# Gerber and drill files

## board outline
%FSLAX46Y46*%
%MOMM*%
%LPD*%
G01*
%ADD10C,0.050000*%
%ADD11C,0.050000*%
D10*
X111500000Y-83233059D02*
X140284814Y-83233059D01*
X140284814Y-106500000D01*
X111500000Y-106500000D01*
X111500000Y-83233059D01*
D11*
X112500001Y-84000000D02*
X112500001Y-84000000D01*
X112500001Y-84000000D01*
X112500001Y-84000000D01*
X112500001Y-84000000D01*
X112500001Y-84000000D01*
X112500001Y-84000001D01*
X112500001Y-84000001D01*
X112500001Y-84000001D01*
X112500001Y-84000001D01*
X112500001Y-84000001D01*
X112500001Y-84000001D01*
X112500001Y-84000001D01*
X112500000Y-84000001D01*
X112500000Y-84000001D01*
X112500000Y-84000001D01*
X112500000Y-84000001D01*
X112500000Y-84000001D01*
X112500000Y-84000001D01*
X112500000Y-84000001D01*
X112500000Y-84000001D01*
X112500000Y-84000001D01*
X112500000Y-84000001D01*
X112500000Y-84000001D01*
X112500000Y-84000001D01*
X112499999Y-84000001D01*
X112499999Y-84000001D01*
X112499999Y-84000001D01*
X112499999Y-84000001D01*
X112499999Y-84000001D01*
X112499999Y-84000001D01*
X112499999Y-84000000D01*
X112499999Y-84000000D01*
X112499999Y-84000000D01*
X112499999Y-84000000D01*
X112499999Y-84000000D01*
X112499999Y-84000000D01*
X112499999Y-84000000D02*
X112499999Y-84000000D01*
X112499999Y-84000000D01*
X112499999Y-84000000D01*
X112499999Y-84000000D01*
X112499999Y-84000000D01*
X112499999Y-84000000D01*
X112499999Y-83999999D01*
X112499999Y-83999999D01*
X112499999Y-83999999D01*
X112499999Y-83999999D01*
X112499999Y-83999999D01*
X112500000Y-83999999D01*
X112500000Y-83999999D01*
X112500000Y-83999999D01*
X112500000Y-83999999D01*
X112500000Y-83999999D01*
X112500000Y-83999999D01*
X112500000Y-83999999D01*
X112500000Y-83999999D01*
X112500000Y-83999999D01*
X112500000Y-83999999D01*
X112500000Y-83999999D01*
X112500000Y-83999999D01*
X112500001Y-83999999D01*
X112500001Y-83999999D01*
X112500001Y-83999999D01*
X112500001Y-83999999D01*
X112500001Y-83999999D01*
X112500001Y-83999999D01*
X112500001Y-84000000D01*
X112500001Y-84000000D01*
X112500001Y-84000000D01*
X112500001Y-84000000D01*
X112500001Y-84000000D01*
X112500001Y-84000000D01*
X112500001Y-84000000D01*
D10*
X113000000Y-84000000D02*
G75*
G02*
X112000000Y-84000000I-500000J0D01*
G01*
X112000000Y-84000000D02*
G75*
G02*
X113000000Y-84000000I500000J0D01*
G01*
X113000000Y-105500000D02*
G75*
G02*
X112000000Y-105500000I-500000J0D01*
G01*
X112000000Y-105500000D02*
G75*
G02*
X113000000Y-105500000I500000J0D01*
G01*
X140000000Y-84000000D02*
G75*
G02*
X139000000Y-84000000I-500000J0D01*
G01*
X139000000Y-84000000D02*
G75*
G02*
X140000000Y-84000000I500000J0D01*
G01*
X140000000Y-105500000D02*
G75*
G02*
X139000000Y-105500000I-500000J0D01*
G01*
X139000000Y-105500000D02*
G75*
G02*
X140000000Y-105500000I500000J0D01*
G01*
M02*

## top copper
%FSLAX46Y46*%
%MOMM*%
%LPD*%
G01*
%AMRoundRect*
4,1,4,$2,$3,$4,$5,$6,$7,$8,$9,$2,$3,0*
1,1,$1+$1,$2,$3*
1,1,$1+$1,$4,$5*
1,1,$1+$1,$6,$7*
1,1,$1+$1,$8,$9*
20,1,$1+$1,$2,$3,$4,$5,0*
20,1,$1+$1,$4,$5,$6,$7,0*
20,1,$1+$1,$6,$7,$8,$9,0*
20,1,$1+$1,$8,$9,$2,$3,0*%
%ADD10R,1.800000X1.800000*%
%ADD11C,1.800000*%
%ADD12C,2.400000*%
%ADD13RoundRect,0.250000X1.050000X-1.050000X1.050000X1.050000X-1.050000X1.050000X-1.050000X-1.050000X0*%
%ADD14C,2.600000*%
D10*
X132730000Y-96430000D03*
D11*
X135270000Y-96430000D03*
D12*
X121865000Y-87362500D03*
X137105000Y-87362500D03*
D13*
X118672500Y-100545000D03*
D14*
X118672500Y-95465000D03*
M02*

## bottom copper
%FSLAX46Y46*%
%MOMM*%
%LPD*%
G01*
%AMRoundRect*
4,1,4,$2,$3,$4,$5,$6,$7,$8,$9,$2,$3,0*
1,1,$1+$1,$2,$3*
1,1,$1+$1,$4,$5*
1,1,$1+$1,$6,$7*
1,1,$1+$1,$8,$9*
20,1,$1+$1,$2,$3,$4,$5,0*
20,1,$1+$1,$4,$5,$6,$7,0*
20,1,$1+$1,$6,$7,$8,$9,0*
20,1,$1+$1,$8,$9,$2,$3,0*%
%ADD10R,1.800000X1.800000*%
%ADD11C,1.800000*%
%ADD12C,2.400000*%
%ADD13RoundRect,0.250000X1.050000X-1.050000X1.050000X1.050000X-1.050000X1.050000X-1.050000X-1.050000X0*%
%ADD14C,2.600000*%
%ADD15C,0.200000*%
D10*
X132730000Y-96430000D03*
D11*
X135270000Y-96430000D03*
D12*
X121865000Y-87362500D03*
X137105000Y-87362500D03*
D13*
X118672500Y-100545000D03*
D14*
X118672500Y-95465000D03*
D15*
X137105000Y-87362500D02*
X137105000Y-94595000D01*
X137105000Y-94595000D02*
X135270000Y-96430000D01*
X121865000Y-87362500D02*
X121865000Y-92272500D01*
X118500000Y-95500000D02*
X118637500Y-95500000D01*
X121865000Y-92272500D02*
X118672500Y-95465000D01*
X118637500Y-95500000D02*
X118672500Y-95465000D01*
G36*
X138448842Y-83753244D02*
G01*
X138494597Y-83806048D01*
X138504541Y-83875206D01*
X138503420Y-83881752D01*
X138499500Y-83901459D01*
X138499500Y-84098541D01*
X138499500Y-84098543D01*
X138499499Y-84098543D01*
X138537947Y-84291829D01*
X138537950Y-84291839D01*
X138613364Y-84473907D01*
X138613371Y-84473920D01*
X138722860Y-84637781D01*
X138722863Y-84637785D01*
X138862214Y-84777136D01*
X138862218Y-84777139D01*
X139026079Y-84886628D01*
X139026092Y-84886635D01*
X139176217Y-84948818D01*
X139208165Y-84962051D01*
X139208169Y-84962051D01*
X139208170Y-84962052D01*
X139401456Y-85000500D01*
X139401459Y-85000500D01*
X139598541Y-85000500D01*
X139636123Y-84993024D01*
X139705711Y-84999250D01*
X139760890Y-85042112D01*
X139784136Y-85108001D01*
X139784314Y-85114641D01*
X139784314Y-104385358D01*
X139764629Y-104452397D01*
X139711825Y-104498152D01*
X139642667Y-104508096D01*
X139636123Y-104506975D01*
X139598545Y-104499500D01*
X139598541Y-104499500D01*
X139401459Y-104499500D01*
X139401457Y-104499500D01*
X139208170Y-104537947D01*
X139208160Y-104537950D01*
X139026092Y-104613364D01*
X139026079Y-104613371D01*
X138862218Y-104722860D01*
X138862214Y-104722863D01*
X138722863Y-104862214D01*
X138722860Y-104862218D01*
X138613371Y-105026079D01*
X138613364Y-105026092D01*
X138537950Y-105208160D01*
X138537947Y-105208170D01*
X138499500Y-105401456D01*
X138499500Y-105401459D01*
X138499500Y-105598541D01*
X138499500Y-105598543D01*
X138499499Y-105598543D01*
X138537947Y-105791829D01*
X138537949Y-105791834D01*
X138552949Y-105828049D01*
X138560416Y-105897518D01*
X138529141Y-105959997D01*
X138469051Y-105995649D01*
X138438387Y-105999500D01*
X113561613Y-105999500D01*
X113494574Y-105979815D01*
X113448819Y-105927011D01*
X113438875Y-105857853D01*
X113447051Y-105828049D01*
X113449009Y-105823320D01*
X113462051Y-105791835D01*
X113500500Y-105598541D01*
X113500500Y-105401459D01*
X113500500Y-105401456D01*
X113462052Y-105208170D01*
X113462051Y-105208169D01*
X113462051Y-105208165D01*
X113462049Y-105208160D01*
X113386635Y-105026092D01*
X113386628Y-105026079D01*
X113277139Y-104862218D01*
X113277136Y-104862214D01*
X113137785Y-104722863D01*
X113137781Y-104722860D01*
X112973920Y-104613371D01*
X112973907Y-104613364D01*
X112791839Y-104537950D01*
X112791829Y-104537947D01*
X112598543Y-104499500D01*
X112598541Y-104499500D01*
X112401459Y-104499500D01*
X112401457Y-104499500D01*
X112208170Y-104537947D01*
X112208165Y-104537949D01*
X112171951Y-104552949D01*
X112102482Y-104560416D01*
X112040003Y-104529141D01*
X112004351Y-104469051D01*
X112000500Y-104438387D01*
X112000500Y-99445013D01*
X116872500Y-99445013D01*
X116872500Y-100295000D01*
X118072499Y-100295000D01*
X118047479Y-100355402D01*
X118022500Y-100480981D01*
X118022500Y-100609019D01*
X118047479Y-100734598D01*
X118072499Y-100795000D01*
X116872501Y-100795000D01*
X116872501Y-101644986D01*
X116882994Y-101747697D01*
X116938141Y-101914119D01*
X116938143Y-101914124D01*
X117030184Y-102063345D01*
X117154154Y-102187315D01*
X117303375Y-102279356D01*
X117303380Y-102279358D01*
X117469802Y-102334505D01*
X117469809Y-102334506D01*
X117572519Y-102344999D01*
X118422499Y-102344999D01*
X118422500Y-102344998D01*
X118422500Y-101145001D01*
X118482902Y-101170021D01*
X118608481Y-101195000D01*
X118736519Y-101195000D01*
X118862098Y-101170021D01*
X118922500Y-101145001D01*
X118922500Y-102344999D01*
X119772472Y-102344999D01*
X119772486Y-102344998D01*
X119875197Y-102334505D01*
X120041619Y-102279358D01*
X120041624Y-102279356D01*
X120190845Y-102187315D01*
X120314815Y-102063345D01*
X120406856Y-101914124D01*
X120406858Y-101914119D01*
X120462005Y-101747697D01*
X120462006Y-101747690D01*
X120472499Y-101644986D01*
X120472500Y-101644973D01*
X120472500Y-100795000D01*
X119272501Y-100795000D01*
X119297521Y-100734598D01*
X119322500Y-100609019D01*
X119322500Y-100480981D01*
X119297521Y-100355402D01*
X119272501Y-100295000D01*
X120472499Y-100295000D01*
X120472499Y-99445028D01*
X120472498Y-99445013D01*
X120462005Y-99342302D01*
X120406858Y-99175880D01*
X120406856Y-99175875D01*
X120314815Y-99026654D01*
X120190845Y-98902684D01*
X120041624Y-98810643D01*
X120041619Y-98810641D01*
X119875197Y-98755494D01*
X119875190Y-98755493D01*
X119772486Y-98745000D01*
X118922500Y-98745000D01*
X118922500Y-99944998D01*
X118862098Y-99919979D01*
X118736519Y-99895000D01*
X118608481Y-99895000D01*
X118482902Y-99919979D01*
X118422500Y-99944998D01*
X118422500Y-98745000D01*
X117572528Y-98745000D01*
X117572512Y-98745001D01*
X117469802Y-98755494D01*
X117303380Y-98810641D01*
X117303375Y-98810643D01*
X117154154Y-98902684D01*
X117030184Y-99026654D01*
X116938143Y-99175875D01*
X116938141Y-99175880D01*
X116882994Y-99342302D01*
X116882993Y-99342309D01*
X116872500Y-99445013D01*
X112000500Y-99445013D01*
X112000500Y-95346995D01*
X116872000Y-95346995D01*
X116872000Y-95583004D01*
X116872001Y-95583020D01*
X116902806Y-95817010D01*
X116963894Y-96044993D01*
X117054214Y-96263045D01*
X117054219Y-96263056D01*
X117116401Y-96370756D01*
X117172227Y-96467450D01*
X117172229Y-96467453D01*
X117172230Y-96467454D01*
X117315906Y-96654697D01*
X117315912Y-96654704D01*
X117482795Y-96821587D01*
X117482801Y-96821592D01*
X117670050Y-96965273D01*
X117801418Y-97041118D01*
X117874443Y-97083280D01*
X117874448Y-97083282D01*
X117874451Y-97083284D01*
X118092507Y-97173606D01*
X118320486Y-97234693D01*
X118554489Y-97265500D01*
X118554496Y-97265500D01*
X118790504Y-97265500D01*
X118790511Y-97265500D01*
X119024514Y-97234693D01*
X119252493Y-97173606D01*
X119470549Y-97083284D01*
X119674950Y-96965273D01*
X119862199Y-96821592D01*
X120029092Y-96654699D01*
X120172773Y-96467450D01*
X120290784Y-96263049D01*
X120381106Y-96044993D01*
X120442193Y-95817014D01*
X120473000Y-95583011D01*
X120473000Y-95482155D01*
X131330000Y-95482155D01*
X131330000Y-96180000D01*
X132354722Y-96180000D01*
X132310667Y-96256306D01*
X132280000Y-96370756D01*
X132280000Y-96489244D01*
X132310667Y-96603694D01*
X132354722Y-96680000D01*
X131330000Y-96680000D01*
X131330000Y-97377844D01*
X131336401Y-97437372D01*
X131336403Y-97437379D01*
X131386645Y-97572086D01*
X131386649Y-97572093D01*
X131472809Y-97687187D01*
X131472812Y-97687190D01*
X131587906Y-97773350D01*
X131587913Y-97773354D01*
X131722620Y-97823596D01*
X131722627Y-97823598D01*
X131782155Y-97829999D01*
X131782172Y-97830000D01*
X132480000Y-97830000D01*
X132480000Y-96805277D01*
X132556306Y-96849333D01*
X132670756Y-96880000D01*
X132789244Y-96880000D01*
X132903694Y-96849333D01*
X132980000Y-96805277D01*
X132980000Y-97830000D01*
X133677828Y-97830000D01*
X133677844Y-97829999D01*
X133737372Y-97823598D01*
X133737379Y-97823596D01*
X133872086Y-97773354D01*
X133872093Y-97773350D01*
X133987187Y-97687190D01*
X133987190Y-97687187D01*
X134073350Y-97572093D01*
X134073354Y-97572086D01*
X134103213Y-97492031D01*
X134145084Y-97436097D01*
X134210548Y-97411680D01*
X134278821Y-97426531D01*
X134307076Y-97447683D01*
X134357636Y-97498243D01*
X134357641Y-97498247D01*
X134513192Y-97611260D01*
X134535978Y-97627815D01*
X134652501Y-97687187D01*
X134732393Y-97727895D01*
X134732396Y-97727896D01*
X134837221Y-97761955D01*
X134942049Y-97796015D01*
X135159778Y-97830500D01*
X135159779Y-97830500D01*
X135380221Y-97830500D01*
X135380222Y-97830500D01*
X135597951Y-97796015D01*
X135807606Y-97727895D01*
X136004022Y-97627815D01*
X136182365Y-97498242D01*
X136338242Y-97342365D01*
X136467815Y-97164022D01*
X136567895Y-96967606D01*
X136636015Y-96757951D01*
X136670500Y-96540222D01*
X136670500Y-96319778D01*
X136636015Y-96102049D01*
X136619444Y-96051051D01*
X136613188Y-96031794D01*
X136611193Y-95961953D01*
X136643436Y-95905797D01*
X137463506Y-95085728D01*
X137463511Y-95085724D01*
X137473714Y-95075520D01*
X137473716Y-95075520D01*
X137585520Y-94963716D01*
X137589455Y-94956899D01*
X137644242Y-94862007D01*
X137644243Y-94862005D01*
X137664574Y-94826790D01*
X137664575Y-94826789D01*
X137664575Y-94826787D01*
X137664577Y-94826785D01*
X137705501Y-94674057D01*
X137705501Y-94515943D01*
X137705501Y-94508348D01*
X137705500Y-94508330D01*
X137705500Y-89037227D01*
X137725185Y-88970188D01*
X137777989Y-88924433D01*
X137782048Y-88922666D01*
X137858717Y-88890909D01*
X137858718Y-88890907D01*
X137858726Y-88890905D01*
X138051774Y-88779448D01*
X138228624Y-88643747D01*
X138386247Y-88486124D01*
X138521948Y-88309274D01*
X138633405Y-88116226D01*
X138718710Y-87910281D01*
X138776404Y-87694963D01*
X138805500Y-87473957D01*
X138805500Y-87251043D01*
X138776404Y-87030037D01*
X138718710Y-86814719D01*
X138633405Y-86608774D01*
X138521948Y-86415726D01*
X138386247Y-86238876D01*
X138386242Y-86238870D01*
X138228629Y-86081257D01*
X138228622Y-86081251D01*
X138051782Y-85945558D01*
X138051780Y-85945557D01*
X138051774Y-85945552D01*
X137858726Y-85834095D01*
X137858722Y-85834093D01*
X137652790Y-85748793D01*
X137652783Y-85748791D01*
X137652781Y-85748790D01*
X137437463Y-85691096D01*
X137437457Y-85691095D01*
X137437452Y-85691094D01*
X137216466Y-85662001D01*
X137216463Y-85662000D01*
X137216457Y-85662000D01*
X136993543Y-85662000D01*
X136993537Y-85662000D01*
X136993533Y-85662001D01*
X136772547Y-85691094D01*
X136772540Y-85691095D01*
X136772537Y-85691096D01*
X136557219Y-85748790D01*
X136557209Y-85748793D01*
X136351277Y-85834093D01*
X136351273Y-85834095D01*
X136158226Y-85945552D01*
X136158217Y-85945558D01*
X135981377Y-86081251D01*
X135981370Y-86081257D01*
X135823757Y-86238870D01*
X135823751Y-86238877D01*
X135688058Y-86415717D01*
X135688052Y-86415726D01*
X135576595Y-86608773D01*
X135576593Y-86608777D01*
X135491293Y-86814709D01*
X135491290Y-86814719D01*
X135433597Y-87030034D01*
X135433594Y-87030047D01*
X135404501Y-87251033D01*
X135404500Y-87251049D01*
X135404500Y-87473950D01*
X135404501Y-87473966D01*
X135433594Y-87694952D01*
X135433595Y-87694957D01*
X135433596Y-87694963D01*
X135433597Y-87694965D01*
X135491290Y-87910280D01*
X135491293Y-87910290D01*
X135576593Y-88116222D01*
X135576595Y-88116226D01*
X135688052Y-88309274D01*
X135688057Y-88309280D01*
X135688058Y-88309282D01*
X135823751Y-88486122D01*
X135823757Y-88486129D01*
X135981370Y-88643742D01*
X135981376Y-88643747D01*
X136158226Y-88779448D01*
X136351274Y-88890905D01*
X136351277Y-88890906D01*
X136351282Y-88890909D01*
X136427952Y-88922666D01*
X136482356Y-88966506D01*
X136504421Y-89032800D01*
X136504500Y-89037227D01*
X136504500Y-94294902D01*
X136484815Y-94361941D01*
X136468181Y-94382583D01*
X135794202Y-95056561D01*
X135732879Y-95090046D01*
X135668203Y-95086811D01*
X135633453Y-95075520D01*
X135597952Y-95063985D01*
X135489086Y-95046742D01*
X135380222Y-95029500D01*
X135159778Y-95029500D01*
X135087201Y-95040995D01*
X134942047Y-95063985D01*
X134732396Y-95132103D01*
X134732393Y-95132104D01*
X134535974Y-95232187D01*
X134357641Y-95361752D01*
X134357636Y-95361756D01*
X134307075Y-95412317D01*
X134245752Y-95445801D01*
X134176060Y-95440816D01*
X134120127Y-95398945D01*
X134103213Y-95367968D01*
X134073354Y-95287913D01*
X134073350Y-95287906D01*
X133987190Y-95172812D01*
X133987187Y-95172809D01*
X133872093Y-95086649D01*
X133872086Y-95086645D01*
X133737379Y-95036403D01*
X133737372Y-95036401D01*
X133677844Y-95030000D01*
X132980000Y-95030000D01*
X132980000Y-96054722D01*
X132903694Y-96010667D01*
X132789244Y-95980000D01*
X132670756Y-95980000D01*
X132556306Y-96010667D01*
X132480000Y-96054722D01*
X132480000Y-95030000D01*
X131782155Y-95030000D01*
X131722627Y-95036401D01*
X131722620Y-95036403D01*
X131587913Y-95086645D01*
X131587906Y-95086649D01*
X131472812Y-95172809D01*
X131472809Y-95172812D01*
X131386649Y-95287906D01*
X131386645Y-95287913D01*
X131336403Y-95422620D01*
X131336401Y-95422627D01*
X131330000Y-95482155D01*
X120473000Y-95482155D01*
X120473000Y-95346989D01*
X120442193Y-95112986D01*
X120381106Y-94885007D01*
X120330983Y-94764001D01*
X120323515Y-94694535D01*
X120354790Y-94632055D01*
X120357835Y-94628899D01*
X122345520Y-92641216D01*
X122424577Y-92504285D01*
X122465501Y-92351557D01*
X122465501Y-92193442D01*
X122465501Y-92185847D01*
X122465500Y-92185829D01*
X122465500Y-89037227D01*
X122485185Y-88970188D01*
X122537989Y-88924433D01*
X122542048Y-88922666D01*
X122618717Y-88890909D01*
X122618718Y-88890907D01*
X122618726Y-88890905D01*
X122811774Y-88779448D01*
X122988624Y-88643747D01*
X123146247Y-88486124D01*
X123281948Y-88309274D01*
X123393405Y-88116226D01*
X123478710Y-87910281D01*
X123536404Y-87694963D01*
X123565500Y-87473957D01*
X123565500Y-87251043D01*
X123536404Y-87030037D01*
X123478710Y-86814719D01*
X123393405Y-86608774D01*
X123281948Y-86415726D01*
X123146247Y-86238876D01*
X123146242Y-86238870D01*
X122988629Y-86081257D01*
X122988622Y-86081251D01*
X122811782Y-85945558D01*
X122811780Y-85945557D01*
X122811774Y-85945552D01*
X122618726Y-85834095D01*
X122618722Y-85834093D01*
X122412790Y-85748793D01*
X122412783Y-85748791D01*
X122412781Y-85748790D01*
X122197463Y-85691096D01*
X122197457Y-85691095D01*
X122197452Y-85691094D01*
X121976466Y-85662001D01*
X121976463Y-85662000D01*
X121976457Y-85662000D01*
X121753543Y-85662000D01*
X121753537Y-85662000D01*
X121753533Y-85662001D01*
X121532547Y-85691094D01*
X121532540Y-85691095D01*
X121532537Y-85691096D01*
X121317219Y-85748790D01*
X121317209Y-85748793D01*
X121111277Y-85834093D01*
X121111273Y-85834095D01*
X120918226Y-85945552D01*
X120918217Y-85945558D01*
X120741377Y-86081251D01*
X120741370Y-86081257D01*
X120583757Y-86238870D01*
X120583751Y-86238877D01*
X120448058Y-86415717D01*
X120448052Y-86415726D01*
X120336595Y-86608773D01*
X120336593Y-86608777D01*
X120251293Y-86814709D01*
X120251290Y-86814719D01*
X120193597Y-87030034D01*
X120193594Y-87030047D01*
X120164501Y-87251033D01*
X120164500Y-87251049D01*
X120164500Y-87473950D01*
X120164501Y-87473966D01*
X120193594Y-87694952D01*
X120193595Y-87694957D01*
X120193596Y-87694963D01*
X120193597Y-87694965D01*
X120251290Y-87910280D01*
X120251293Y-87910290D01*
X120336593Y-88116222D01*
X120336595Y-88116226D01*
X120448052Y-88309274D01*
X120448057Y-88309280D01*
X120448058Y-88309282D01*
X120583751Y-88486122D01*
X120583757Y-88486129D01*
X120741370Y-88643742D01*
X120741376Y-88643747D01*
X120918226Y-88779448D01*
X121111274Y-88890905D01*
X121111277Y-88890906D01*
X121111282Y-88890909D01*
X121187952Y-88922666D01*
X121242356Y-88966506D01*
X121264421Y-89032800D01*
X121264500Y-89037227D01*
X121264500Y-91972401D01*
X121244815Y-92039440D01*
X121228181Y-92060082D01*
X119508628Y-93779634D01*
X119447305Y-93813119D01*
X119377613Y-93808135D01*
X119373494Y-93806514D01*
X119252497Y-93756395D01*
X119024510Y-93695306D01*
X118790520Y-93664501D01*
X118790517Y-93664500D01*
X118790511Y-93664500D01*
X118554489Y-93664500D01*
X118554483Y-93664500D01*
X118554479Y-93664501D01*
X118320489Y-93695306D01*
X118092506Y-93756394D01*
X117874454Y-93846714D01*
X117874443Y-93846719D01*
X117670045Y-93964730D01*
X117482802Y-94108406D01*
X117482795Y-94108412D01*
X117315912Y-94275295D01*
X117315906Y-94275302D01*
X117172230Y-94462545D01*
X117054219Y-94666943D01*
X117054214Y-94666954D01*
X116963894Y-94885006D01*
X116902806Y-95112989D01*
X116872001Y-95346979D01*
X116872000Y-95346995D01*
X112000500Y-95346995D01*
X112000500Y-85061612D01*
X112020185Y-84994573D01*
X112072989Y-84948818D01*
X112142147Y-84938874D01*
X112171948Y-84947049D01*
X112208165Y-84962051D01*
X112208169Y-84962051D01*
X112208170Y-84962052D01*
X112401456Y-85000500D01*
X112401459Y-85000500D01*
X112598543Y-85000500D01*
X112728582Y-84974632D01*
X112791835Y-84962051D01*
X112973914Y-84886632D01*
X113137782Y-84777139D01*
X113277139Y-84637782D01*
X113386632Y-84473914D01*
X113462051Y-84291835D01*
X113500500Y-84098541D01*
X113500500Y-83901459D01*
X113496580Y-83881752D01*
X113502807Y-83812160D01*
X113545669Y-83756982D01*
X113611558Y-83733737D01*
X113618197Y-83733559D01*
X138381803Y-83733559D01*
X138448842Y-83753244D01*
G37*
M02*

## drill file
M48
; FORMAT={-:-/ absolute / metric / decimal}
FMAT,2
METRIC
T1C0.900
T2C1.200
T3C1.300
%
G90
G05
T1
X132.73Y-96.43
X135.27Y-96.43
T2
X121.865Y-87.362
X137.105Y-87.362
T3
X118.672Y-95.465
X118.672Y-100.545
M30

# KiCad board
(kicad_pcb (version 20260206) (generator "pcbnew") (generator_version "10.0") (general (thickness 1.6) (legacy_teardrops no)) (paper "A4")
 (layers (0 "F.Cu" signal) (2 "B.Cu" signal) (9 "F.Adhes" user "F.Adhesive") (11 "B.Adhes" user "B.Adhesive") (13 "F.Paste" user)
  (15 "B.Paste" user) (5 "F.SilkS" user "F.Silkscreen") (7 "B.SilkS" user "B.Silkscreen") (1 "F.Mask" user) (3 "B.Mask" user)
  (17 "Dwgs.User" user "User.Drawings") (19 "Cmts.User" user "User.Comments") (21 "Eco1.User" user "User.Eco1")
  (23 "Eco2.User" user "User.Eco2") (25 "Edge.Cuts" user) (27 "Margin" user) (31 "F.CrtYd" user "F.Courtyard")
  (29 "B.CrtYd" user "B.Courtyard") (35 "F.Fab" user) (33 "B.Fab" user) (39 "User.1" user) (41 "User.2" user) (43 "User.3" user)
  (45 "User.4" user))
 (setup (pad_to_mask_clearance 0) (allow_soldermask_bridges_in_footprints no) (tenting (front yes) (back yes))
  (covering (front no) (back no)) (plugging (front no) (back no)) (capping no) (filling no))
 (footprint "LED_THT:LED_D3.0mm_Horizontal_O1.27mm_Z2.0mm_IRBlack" (layer "F.Cu") (at 132.73 96.43)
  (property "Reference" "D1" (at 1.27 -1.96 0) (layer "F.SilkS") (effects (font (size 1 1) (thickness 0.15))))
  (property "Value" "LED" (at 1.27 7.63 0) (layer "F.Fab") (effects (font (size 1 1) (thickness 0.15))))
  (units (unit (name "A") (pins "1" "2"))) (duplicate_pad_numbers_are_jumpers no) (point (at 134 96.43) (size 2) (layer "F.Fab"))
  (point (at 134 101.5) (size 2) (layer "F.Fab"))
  (pad "1" thru_hole rect (at 0 0) (size 1.8 1.8) (drill 0.9) (layers "*.Cu" "*.Mask") (remove_unused_layers no) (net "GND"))
  (pad "2" thru_hole circle (at 2.54 0) (size 1.8 1.8) (drill 0.9) (layers "*.Cu" "*.Mask") (remove_unused_layers no) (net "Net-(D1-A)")))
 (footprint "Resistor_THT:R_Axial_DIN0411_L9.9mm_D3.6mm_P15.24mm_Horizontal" (layer "F.Cu") (at 121.865 87.3625)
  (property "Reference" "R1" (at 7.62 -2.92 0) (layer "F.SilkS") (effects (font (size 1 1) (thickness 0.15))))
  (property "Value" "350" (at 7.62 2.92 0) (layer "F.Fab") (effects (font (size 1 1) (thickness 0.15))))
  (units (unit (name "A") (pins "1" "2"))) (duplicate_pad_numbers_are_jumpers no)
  (pad "1" thru_hole circle (at 0 0) (size 2.4 2.4) (drill 1.2) (layers "*.Cu" "*.Mask") (remove_unused_layers no) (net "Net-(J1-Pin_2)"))
  (pad "2" thru_hole circle (at 15.24 0) (size 2.4 2.4) (drill 1.2) (layers "*.Cu" "*.Mask") (remove_unused_layers no) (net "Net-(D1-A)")))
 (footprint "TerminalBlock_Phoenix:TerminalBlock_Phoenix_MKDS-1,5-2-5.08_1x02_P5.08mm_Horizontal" (layer "F.Cu") (at 118.6725 100.545 90)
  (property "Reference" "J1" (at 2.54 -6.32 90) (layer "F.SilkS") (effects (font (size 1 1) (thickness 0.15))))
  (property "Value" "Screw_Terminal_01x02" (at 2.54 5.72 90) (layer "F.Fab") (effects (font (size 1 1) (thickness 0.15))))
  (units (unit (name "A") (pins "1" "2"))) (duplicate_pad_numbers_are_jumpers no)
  (pad "1" thru_hole roundrect (at 0 0 90) (size 2.6 2.6) (drill 1.3) (layers "*.Cu" "*.Mask") (remove_unused_layers no)
   (roundrect_rratio 0.096154) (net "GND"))
  (pad "2" thru_hole circle (at 5.08 0 90) (size 2.6 2.6) (drill 1.3) (layers "*.Cu" "*.Mask") (remove_unused_layers no)
   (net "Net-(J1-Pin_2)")))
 (gr_rect (start 111.5 83.233059) (end 140.284814 106.5) (stroke (width 0.05) (type default)) (fill no) (layer "Edge.Cuts"))
 (gr_circle (center 112.5 84) (end 112.5 84) (stroke (width 0.05) (type default)) (fill no) (layer "Edge.Cuts"))
 (gr_circle (center 112.5 84) (end 113 84) (stroke (width 0.05) (type default)) (fill no) (layer "Edge.Cuts"))
 (gr_circle (center 112.5 105.5) (end 113 105.5) (stroke (width 0.05) (type default)) (fill no) (layer "Edge.Cuts"))
 (gr_circle (center 139.5 84) (end 139.5 84.5) (stroke (width 0.05) (type default)) (fill no) (layer "Edge.Cuts"))
 (gr_circle (center 139.5 105.5) (end 139.5 106) (stroke (width 0.05) (type default)) (fill no) (layer "Edge.Cuts"))
 (segment (start 137.105 87.3625) (end 137.105 94.595) (width 0.2) (layer "B.Cu") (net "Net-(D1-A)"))
 (segment (start 137.105 94.595) (end 135.27 96.43) (width 0.2) (layer "B.Cu") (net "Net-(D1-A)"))
 (segment (start 121.865 87.3625) (end 121.865 92.2725) (width 0.2) (layer "B.Cu") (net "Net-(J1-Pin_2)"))
 (segment (start 118.5 95.5) (end 118.6375 95.5) (width 0.2) (layer "B.Cu") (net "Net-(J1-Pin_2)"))
 (segment (start 121.865 92.2725) (end 118.6725 95.465) (width 0.2) (layer "B.Cu") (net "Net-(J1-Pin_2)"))
 (segment (start 118.6375 95.5) (end 118.6725 95.465) (width 0.2) (layer "B.Cu") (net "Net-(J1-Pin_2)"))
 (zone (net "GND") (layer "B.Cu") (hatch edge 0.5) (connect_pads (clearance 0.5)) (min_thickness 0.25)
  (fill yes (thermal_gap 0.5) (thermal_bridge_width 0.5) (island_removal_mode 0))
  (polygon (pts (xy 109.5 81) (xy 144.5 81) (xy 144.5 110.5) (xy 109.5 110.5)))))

